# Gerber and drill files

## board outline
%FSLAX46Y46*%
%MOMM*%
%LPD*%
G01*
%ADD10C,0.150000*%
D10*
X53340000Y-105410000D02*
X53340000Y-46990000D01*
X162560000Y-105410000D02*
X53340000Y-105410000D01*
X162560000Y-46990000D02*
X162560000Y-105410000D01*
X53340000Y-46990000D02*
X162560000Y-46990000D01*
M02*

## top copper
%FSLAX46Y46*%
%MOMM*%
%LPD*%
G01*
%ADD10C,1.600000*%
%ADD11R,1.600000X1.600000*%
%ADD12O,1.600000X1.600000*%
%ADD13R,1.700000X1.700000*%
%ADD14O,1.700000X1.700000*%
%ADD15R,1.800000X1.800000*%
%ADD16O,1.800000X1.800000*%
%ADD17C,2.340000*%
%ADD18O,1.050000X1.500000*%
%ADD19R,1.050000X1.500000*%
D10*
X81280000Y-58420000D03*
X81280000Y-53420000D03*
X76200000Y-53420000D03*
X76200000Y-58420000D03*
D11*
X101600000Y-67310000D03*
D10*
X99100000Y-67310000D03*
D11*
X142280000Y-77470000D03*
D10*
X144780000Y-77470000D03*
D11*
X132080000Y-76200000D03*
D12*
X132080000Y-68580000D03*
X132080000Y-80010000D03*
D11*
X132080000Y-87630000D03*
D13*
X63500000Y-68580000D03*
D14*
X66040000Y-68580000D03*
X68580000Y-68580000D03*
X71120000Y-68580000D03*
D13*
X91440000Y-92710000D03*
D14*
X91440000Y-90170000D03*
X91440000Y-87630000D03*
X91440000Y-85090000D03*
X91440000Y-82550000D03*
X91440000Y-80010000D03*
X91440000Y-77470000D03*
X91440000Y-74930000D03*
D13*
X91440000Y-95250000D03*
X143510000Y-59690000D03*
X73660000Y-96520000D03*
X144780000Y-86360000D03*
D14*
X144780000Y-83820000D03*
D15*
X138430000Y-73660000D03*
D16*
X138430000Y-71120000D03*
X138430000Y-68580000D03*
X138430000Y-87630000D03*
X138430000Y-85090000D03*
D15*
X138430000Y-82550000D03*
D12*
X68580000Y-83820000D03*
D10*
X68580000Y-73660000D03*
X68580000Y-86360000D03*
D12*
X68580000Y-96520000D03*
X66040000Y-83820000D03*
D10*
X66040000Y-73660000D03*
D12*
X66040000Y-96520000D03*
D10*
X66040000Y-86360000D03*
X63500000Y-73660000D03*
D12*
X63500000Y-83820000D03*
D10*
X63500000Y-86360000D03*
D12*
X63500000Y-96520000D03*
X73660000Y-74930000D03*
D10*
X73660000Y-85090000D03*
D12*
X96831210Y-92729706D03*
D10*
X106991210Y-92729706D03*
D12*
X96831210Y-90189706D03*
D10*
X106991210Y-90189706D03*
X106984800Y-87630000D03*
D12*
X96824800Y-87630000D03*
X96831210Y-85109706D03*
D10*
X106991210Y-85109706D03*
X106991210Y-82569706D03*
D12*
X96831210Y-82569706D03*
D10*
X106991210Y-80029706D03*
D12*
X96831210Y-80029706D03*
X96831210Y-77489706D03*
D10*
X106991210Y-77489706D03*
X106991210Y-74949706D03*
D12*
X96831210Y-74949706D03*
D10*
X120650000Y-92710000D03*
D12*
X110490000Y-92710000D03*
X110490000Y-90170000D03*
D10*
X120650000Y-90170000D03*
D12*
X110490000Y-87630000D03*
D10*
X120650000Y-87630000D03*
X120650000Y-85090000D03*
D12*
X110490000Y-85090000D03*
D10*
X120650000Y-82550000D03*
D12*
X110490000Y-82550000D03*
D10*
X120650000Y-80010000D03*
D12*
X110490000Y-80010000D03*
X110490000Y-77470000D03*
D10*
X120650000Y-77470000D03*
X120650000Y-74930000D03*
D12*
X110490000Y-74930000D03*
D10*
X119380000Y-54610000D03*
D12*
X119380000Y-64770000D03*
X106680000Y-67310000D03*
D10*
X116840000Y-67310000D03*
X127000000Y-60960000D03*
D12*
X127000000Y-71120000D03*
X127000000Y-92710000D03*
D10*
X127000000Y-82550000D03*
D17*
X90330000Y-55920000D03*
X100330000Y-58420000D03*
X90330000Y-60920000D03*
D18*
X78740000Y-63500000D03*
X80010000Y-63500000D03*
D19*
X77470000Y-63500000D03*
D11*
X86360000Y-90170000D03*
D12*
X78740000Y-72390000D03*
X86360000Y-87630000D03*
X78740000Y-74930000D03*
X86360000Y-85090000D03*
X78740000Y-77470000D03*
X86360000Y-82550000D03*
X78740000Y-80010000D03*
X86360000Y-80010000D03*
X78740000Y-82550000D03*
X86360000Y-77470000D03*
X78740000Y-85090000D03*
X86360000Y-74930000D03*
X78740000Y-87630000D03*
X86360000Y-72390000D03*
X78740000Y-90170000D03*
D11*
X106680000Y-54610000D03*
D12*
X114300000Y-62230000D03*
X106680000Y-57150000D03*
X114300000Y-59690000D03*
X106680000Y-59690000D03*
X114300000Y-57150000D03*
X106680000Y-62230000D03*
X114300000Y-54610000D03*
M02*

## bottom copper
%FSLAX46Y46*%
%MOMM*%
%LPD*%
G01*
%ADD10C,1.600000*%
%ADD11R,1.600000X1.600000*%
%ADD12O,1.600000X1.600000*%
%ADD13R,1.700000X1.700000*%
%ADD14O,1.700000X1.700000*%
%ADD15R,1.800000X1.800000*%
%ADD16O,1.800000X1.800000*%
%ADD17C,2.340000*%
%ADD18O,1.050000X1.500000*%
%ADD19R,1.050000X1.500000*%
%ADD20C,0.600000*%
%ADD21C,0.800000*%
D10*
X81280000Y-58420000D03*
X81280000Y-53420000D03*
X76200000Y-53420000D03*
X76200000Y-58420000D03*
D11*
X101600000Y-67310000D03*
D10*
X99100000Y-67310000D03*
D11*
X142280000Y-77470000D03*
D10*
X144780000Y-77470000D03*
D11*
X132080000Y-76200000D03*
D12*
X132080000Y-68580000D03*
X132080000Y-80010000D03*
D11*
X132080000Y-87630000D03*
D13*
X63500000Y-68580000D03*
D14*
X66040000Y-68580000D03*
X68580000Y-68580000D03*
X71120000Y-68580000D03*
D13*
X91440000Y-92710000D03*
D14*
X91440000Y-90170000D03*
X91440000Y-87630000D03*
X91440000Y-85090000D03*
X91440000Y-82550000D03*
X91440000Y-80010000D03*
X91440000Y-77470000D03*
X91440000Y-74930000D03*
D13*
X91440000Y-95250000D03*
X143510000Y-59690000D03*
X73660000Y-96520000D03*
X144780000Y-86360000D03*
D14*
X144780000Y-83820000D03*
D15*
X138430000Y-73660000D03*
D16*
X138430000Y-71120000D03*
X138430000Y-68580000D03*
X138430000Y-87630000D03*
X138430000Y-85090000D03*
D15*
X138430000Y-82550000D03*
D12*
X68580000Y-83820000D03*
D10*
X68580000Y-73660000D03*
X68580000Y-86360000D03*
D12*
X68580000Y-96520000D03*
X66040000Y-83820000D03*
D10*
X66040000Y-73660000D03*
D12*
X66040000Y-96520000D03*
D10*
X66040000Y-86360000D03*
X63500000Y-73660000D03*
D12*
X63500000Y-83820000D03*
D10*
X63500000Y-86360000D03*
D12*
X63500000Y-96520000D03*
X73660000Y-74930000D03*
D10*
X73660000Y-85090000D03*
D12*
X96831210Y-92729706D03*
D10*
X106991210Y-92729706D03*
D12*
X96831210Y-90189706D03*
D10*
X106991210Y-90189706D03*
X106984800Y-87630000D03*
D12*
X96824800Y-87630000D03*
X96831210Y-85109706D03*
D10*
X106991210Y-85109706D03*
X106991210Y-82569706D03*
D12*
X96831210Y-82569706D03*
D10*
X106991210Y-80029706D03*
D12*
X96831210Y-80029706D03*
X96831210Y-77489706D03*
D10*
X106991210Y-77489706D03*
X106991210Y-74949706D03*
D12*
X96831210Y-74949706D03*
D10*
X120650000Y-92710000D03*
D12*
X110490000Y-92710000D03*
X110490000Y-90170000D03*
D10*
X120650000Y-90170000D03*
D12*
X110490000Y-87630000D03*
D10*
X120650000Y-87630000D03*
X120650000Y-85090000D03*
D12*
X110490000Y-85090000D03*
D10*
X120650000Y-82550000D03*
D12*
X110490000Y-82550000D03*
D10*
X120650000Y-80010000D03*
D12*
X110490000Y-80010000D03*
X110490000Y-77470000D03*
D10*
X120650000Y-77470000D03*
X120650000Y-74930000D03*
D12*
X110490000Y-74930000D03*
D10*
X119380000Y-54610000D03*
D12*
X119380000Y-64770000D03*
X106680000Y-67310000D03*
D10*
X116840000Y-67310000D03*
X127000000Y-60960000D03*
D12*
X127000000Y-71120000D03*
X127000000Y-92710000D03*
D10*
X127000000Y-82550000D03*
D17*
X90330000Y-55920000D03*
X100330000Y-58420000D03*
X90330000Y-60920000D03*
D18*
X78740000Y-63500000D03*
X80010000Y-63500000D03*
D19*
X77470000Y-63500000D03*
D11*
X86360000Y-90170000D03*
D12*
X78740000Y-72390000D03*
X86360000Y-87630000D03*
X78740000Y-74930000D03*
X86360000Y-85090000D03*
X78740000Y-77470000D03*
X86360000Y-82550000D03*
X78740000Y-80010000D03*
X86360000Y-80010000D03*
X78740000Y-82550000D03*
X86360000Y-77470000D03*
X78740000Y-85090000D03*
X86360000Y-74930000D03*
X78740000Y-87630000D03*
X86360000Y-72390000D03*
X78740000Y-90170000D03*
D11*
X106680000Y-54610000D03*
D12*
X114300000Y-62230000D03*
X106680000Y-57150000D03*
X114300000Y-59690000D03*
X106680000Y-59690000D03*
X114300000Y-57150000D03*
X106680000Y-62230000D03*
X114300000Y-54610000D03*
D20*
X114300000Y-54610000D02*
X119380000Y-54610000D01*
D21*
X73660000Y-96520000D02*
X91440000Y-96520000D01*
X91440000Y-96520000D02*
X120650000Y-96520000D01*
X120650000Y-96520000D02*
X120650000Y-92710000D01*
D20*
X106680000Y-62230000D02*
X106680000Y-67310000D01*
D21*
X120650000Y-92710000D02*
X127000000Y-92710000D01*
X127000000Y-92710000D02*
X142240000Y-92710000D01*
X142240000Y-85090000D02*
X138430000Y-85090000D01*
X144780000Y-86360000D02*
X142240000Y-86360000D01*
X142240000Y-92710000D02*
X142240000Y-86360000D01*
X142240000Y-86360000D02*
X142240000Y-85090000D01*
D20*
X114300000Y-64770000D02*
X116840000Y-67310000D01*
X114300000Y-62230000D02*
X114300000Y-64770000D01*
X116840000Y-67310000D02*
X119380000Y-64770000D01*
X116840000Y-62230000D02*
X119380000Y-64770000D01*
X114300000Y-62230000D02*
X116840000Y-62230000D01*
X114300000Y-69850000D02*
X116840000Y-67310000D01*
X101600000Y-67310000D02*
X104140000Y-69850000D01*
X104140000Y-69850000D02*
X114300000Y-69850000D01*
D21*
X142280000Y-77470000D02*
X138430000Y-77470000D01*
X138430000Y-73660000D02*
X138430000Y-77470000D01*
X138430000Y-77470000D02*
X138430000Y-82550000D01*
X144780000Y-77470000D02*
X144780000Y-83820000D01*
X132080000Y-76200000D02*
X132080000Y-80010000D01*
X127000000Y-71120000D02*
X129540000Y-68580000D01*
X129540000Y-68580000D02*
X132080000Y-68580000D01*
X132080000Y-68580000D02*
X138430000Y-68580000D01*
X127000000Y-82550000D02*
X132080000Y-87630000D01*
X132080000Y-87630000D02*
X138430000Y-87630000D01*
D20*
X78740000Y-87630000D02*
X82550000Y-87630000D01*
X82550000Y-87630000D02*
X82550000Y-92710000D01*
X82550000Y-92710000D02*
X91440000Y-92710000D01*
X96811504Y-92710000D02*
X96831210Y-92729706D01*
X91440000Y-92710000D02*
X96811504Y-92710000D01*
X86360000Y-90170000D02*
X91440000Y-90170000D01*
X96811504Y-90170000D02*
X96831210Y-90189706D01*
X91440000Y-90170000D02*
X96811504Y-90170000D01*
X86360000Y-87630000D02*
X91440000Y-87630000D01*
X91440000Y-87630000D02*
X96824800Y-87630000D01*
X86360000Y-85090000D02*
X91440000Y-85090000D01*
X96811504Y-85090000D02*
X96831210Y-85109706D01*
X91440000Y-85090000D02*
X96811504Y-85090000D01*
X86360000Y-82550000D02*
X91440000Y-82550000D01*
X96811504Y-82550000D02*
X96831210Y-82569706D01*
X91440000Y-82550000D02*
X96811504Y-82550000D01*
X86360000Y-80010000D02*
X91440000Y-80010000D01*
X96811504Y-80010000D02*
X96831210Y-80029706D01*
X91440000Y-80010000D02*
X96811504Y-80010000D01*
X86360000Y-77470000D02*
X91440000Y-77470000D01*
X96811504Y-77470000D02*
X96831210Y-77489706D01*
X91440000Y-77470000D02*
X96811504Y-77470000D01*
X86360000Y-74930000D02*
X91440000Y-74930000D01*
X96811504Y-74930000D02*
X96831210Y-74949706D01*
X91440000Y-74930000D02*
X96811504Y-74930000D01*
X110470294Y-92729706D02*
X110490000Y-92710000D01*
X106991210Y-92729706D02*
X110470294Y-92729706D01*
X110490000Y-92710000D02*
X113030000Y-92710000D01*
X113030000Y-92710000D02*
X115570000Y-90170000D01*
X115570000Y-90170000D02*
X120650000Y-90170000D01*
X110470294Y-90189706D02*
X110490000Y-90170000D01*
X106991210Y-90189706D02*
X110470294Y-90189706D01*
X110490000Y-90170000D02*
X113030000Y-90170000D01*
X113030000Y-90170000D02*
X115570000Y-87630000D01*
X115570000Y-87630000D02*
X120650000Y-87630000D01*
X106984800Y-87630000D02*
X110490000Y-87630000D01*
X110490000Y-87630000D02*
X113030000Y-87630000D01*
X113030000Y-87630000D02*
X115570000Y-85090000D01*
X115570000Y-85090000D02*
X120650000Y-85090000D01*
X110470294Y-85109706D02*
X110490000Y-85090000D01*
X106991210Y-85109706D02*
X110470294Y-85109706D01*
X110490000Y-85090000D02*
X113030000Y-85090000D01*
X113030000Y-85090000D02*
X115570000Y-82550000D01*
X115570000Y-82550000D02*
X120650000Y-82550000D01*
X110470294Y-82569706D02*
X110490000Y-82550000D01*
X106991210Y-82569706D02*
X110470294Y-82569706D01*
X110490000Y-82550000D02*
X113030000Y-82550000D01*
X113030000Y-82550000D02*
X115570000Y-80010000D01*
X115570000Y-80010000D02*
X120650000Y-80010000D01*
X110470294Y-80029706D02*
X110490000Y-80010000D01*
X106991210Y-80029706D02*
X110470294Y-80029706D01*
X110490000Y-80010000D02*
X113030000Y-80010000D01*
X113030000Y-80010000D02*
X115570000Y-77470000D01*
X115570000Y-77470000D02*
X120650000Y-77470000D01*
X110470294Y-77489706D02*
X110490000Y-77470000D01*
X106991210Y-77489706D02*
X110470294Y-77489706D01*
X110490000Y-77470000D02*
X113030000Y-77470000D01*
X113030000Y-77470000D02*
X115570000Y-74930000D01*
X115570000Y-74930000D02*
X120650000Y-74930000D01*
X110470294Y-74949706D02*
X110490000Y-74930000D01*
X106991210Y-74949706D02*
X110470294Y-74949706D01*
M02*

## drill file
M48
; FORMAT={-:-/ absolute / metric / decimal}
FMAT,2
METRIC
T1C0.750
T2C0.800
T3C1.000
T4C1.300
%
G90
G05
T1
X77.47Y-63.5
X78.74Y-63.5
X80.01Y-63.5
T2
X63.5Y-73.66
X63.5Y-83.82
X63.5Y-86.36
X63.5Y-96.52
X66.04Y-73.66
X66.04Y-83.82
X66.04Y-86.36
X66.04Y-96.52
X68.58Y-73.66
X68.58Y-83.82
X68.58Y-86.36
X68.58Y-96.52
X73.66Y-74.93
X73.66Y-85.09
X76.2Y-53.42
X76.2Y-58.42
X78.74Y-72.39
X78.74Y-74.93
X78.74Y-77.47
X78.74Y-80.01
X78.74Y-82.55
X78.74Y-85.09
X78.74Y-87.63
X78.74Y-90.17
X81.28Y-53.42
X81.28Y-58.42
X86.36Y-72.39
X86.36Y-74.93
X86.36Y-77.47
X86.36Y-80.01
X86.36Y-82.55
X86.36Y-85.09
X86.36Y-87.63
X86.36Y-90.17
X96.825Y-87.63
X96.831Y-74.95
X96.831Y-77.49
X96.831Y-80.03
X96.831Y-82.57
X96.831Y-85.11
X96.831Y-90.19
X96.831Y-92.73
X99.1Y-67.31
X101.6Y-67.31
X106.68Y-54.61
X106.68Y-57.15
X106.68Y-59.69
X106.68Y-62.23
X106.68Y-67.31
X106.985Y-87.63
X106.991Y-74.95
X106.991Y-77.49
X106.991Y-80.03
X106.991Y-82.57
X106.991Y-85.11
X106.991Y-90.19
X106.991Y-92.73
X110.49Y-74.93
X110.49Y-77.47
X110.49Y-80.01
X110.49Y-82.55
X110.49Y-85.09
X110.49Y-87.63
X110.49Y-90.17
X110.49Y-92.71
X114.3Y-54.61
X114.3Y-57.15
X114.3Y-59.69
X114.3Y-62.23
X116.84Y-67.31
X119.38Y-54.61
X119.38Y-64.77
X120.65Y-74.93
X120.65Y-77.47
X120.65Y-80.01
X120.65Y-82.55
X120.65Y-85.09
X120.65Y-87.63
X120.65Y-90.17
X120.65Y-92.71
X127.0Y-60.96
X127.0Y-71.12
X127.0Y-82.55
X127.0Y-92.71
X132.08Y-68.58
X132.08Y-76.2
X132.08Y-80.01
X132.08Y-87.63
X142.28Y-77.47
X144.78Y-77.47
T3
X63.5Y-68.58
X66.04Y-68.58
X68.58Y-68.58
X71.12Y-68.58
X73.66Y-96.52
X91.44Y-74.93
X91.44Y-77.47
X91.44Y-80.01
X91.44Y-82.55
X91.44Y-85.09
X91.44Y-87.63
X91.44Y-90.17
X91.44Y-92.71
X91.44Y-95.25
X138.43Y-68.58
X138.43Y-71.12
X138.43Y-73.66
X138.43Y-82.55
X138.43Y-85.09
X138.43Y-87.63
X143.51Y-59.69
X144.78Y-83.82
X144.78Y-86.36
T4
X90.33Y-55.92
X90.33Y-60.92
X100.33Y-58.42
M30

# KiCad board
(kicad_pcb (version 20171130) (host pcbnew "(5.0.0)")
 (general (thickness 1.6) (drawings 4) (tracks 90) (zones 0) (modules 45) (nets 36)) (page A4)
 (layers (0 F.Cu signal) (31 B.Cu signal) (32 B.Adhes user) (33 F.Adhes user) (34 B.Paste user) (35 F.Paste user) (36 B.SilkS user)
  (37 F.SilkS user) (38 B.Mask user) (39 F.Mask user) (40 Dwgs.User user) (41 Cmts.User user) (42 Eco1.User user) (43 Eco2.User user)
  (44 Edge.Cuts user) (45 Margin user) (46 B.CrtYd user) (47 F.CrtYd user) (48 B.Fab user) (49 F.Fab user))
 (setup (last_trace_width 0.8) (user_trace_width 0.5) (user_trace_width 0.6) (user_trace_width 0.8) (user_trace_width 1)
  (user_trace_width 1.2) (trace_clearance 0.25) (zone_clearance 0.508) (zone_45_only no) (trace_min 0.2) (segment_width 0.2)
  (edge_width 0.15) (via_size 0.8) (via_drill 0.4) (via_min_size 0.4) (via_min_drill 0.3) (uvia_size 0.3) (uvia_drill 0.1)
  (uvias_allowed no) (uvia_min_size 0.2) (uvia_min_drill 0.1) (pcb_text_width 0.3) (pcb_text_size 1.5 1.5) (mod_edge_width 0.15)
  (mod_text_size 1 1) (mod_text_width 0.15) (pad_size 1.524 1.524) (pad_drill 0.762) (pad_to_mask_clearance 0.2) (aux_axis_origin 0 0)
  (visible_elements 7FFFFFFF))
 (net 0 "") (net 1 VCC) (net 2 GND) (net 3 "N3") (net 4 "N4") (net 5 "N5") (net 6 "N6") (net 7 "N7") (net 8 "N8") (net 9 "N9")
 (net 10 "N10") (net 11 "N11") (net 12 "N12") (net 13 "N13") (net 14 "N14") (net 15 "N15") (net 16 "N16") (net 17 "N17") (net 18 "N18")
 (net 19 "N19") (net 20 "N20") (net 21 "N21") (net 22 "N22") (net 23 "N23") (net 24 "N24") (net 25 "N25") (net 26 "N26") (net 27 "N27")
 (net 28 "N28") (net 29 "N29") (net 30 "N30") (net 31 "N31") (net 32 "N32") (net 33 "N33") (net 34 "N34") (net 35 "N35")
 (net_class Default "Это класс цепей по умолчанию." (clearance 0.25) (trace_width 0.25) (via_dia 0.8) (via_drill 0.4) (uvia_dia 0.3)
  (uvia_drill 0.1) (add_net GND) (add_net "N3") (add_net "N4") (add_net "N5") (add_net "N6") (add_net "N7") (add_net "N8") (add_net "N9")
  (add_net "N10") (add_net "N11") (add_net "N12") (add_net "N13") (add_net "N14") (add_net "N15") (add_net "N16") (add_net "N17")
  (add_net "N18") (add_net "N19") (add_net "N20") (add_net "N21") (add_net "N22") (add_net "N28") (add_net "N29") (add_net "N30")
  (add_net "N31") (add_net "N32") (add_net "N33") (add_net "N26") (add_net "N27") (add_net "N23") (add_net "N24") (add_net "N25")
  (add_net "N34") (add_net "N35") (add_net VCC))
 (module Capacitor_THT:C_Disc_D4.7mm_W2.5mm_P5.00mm (layer F.Cu) (at 81.28 58.42 90)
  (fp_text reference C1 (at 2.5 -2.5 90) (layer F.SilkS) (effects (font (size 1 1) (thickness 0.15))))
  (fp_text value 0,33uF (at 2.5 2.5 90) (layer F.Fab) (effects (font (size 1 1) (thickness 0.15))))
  (pad 1 thru_hole circle (at 0 0 90) (size 1.6 1.6) (drill 0.8) (layers *.Cu *.Mask) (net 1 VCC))
  (pad 2 thru_hole circle (at 5 0 90) (size 1.6 1.6) (drill 0.8) (layers *.Cu *.Mask) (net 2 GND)))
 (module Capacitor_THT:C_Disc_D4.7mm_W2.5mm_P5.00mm (layer F.Cu) (at 76.2 58.42 90)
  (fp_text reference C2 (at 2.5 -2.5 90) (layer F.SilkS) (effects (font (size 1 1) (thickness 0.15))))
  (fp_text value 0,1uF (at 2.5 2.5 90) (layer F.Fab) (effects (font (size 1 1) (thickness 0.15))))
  (pad 2 thru_hole circle (at 5 0 90) (size 1.6 1.6) (drill 0.8) (layers *.Cu *.Mask) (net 2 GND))
  (pad 1 thru_hole circle (at 0 0 90) (size 1.6 1.6) (drill 0.8) (layers *.Cu *.Mask) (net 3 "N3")))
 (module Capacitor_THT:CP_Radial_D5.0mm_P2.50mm (layer F.Cu) (at 101.6 67.31 180)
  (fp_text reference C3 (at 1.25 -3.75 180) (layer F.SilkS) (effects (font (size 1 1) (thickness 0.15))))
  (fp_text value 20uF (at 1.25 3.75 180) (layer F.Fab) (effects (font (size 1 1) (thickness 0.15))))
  (pad 1 thru_hole rect (at 0 0 180) (size 1.6 1.6) (drill 0.8) (layers *.Cu *.Mask) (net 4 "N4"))
  (pad 2 thru_hole circle (at 2.5 0 180) (size 1.6 1.6) (drill 0.8) (layers *.Cu *.Mask) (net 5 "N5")))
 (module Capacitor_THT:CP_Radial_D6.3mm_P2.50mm (layer F.Cu) (at 142.28 77.47)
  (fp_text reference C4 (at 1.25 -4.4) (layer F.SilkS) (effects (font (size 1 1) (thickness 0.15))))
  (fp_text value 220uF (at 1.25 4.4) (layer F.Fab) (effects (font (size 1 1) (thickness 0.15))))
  (pad 1 thru_hole rect (at 0 0) (size 1.6 1.6) (drill 0.8) (layers *.Cu *.Mask) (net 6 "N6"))
  (pad 2 thru_hole circle (at 2.5 0) (size 1.6 1.6) (drill 0.8) (layers *.Cu *.Mask) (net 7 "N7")))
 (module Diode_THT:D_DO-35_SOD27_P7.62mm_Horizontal (layer F.Cu) (at 132.08 76.2 90)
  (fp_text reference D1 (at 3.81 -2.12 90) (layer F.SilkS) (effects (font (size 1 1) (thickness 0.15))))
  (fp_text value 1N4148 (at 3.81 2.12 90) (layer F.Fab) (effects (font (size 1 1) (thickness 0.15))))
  (pad 1 thru_hole rect (at 0 0 90) (size 1.6 1.6) (drill 0.8) (layers *.Cu *.Mask) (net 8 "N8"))
  (pad 2 thru_hole oval (at 7.62 0 90) (size 1.6 1.6) (drill 0.8) (layers *.Cu *.Mask) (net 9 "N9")))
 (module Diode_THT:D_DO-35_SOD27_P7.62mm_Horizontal (layer F.Cu) (at 132.08 87.63 90)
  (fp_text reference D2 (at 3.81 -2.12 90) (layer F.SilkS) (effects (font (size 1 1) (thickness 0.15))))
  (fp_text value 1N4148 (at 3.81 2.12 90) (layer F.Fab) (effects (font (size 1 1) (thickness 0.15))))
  (pad 2 thru_hole oval (at 7.62 0 90) (size 1.6 1.6) (drill 0.8) (layers *.Cu *.Mask) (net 8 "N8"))
  (pad 1 thru_hole rect (at 0 0 90) (size 1.6 1.6) (drill 0.8) (layers *.Cu *.Mask) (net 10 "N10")))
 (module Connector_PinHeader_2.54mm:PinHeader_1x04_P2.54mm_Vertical (layer F.Cu) (at 63.5 68.58 90)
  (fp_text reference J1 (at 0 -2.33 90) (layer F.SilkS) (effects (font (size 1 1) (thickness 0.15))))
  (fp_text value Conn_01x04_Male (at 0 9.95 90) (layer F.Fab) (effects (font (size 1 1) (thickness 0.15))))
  (pad 1 thru_hole rect (at 0 0 90) (size 1.7 1.7) (drill 1) (layers *.Cu *.Mask) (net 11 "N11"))
  (pad 2 thru_hole oval (at 0 2.54 90) (size 1.7 1.7) (drill 1) (layers *.Cu *.Mask) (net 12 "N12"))
  (pad 3 thru_hole oval (at 0 5.08 90) (size 1.7 1.7) (drill 1) (layers *.Cu *.Mask) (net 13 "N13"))
  (pad 4 thru_hole oval (at 0 7.62 90) (size 1.7 1.7) (drill 1) (layers *.Cu *.Mask) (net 2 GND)))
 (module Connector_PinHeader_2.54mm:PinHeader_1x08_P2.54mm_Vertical (layer F.Cu) (at 91.44 92.71 180)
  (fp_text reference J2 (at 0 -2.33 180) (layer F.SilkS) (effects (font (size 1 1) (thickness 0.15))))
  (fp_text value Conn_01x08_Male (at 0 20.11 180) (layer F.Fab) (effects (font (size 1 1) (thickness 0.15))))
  (pad 1 thru_hole rect (at 0 0 180) (size 1.7 1.7) (drill 1) (layers *.Cu *.Mask) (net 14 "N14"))
  (pad 2 thru_hole oval (at 0 2.54 180) (size 1.7 1.7) (drill 1) (layers *.Cu *.Mask) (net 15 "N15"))
  (pad 3 thru_hole oval (at 0 5.08 180) (size 1.7 1.7) (drill 1) (layers *.Cu *.Mask) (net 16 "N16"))
  (pad 4 thru_hole oval (at 0 7.62 180) (size 1.7 1.7) (drill 1) (layers *.Cu *.Mask) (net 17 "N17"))
  (pad 5 thru_hole oval (at 0 10.16 180) (size 1.7 1.7) (drill 1) (layers *.Cu *.Mask) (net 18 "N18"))
  (pad 6 thru_hole oval (at 0 12.7 180) (size 1.7 1.7) (drill 1) (layers *.Cu *.Mask) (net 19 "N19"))
  (pad 7 thru_hole oval (at 0 15.24 180) (size 1.7 1.7) (drill 1) (layers *.Cu *.Mask) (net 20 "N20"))
  (pad 8 thru_hole oval (at 0 17.78 180) (size 1.7 1.7) (drill 1) (layers *.Cu *.Mask) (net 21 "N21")))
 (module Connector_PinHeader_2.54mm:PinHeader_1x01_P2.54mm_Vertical (layer F.Cu) (at 91.44 95.25)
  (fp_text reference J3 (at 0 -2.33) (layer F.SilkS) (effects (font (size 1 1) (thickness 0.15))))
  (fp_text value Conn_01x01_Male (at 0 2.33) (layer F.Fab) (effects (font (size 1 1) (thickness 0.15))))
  (pad 1 thru_hole rect (at 0 0) (size 1.7 1.7) (drill 1) (layers *.Cu *.Mask) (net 2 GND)))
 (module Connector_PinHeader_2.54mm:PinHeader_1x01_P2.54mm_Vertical (layer F.Cu) (at 143.51 59.69)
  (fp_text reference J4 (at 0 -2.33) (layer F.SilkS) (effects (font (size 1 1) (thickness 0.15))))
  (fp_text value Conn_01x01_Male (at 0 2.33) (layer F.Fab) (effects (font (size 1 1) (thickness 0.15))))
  (pad 1 thru_hole rect (at 0 0) (size 1.7 1.7) (drill 1) (layers *.Cu *.Mask) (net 1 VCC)))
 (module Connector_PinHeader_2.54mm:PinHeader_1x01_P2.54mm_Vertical (layer F.Cu) (at 73.66 96.52)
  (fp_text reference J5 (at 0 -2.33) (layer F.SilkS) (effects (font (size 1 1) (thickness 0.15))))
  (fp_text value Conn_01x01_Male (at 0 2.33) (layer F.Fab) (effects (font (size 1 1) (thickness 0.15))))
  (pad 1 thru_hole rect (at 0 0) (size 1.7 1.7) (drill 1) (layers *.Cu *.Mask) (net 2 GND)))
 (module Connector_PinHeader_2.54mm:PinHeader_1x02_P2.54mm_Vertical (layer F.Cu) (at 144.78 86.36 180)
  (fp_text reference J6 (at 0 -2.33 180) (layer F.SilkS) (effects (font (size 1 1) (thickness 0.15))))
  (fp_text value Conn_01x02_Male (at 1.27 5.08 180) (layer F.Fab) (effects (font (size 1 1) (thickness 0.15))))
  (pad 1 thru_hole rect (at 0 0 180) (size 1.7 1.7) (drill 1) (layers *.Cu *.Mask) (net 2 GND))
  (pad 2 thru_hole oval (at 0 2.54 180) (size 1.7 1.7) (drill 1) (layers *.Cu *.Mask) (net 7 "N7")))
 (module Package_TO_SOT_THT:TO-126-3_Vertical (layer F.Cu) (at 138.43 73.66 90)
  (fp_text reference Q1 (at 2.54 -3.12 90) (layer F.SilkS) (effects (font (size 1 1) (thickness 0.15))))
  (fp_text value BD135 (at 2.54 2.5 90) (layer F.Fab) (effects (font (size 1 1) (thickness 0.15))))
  (pad 1 thru_hole rect (at 0 0 90) (size 1.8 1.8) (drill 1) (layers *.Cu *.Mask) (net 6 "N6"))
  (pad 2 thru_hole oval (at 2.54 0 90) (size 1.8 1.8) (drill 1) (layers *.Cu *.Mask) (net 1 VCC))
  (pad 3 thru_hole oval (at 5.08 0 90) (size 1.8 1.8) (drill 1) (layers *.Cu *.Mask) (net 9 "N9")))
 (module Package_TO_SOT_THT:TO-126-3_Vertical (layer F.Cu) (at 138.43 82.55 270)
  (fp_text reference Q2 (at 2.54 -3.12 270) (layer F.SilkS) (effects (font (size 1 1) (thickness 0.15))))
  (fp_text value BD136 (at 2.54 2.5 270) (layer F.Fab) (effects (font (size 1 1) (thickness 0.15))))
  (pad 3 thru_hole oval (at 5.08 0 270) (size 1.8 1.8) (drill 1) (layers *.Cu *.Mask) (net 10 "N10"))
  (pad 2 thru_hole oval (at 2.54 0 270) (size 1.8 1.8) (drill 1) (layers *.Cu *.Mask) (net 2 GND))
  (pad 1 thru_hole rect (at 0 0 270) (size 1.8 1.8) (drill 1) (layers *.Cu *.Mask) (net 6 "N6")))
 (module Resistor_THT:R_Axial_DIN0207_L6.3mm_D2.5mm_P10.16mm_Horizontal (layer F.Cu) (at 68.58 73.66 270)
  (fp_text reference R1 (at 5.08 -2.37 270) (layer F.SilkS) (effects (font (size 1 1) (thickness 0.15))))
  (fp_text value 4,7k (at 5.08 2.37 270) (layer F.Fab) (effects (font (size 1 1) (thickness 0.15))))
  (pad 2 thru_hole oval (at 10.16 0 270) (size 1.6 1.6) (drill 0.8) (layers *.Cu *.Mask) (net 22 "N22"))
  (pad 1 thru_hole circle (at 0 0 270) (size 1.6 1.6) (drill 0.8) (layers *.Cu *.Mask) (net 13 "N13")))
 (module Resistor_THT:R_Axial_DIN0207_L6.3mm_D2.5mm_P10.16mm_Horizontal (layer F.Cu) (at 68.58 86.36 270)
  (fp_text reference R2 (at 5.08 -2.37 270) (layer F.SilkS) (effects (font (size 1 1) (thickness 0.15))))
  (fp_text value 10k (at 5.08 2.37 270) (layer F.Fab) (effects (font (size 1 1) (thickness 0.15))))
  (pad 1 thru_hole circle (at 0 0 270) (size 1.6 1.6) (drill 0.8) (layers *.Cu *.Mask) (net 22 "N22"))
  (pad 2 thru_hole oval (at 10.16 0 270) (size 1.6 1.6) (drill 0.8) (layers *.Cu *.Mask) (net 2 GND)))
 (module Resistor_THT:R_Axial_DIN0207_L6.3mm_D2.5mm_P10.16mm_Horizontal (layer F.Cu) (at 66.04 73.66 270)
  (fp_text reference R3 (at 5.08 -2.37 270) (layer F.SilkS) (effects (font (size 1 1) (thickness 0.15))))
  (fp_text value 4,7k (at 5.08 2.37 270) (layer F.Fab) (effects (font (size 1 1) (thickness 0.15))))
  (pad 2 thru_hole oval (at 10.16 0 270) (size 1.6 1.6) (drill 0.8) (layers *.Cu *.Mask) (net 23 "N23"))
  (pad 1 thru_hole circle (at 0 0 270) (size 1.6 1.6) (drill 0.8) (layers *.Cu *.Mask) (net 12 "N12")))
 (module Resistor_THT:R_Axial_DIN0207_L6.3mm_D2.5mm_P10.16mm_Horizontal (layer F.Cu) (at 66.04 86.36 270)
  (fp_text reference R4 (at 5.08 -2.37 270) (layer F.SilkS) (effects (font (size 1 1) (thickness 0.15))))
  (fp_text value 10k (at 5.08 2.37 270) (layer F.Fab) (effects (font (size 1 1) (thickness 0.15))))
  (pad 2 thru_hole oval (at 10.16 0 270) (size 1.6 1.6) (drill 0.8) (layers *.Cu *.Mask) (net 2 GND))
  (pad 1 thru_hole circle (at 0 0 270) (size 1.6 1.6) (drill 0.8) (layers *.Cu *.Mask) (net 23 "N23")))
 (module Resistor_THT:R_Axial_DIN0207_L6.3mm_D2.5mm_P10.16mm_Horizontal (layer F.Cu) (at 63.5 73.66 270)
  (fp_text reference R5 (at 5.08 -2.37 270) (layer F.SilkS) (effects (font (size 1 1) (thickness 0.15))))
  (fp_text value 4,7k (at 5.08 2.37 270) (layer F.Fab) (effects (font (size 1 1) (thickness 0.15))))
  (pad 1 thru_hole circle (at 0 0 270) (size 1.6 1.6) (drill 0.8) (layers *.Cu *.Mask) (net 11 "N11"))
  (pad 2 thru_hole oval (at 10.16 0 270) (size 1.6 1.6) (drill 0.8) (layers *.Cu *.Mask) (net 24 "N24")))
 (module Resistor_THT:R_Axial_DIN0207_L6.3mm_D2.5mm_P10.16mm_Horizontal (layer F.Cu) (at 63.5 86.36 270)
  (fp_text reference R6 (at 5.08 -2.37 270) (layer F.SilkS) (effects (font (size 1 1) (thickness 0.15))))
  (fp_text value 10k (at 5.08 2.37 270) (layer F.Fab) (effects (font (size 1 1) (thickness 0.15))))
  (pad 1 thru_hole circle (at 0 0 270) (size 1.6 1.6) (drill 0.8) (layers *.Cu *.Mask) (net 24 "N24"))
  (pad 2 thru_hole oval (at 10.16 0 270) (size 1.6 1.6) (drill 0.8) (layers *.Cu *.Mask) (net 2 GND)))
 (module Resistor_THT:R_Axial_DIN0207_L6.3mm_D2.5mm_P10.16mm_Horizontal (layer F.Cu) (at 73.66 85.09 90)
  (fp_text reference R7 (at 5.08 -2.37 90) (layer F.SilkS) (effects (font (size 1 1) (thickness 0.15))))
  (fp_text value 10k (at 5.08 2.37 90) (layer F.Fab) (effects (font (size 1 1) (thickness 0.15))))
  (pad 2 thru_hole oval (at 10.16 0 90) (size 1.6 1.6) (drill 0.8) (layers *.Cu *.Mask) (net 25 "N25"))
  (pad 1 thru_hole circle (at 0 0 90) (size 1.6 1.6) (drill 0.8) (layers *.Cu *.Mask) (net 3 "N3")))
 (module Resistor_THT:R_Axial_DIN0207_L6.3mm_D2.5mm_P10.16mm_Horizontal (layer F.Cu) (at 106.99121 92.729706 180)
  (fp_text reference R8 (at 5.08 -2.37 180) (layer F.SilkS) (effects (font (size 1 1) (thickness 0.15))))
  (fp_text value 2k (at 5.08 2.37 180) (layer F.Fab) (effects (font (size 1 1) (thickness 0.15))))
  (pad 2 thru_hole oval (at 10.16 0 180) (size 1.6 1.6) (drill 0.8) (layers *.Cu *.Mask) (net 14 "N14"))
  (pad 1 thru_hole circle (at 0 0 180) (size 1.6 1.6) (drill 0.8) (layers *.Cu *.Mask) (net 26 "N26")))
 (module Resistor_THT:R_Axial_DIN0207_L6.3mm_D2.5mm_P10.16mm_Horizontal (layer F.Cu) (at 106.99121 90.189706 180)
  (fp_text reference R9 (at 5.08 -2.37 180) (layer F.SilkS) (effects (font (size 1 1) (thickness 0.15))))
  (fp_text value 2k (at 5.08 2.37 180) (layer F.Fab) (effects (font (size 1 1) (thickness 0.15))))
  (pad 2 thru_hole oval (at 10.16 0 180) (size 1.6 1.6) (drill 0.8) (layers *.Cu *.Mask) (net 15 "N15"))
  (pad 1 thru_hole circle (at 0 0 180) (size 1.6 1.6) (drill 0.8) (layers *.Cu *.Mask) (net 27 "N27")))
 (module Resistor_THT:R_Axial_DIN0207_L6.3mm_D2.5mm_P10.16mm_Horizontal (layer F.Cu) (at 106.9848 87.63 180)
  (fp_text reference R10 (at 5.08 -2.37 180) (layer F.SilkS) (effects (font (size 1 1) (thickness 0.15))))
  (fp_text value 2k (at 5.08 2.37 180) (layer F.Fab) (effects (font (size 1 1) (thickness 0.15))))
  (pad 1 thru_hole circle (at 0 0 180) (size 1.6 1.6) (drill 0.8) (layers *.Cu *.Mask) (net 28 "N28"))
  (pad 2 thru_hole oval (at 10.16 0 180) (size 1.6 1.6) (drill 0.8) (layers *.Cu *.Mask) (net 16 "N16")))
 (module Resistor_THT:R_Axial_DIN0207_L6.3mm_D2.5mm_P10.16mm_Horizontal (layer F.Cu) (at 106.99121 85.109706 180)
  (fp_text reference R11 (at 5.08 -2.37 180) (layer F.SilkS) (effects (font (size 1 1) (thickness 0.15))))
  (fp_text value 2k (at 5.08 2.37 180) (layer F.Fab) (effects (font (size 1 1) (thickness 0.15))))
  (pad 2 thru_hole oval (at 10.16 0 180) (size 1.6 1.6) (drill 0.8) (layers *.Cu *.Mask) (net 17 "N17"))
  (pad 1 thru_hole circle (at 0 0 180) (size 1.6 1.6) (drill 0.8) (layers *.Cu *.Mask) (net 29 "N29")))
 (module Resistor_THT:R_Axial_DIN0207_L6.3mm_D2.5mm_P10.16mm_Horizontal (layer F.Cu) (at 106.99121 82.569706 180)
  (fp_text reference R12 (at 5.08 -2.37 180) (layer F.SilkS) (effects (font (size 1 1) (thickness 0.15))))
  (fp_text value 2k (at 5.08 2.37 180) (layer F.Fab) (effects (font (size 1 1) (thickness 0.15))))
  (pad 1 thru_hole circle (at 0 0 180) (size 1.6 1.6) (drill 0.8) (layers *.Cu *.Mask) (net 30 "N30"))
  (pad 2 thru_hole oval (at 10.16 0 180) (size 1.6 1.6) (drill 0.8) (layers *.Cu *.Mask) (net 18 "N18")))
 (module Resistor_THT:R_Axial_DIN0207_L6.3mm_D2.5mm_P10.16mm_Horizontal (layer F.Cu) (at 106.99121 80.029706 180)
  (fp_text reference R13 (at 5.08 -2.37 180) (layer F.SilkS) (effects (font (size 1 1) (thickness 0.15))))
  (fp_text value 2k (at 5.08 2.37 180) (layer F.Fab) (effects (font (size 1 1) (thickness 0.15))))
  (pad 1 thru_hole circle (at 0 0 180) (size 1.6 1.6) (drill 0.8) (layers *.Cu *.Mask) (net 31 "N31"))
  (pad 2 thru_hole oval (at 10.16 0 180) (size 1.6 1.6) (drill 0.8) (layers *.Cu *.Mask) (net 19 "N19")))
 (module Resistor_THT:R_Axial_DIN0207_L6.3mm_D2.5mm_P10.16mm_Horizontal (layer F.Cu) (at 106.99121 77.489706 180)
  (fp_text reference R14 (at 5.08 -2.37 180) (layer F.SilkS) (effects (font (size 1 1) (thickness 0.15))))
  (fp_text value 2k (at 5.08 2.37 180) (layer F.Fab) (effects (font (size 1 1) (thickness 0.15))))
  (pad 2 thru_hole oval (at 10.16 0 180) (size 1.6 1.6) (drill 0.8) (layers *.Cu *.Mask) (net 20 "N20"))
  (pad 1 thru_hole circle (at 0 0 180) (size 1.6 1.6) (drill 0.8) (layers *.Cu *.Mask) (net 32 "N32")))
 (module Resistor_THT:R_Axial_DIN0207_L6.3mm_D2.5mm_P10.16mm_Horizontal (layer F.Cu) (at 106.99121 74.949706 180)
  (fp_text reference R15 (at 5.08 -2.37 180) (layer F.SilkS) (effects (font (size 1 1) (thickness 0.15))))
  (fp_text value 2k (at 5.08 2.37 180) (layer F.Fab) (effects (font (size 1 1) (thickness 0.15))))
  (pad 1 thru_hole circle (at 0 0 180) (size 1.6 1.6) (drill 0.8) (layers *.Cu *.Mask) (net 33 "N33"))
  (pad 2 thru_hole oval (at 10.16 0 180) (size 1.6 1.6) (drill 0.8) (layers *.Cu *.Mask) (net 21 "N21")))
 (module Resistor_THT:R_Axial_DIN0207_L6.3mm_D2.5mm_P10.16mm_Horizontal (layer F.Cu) (at 120.65 92.71 180)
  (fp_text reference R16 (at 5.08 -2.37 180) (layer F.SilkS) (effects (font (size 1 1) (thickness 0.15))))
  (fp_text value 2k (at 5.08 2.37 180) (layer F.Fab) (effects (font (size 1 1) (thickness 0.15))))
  (pad 1 thru_hole circle (at 0 0 180) (size 1.6 1.6) (drill 0.8) (layers *.Cu *.Mask) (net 2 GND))
  (pad 2 thru_hole oval (at 10.16 0 180) (size 1.6 1.6) (drill 0.8) (layers *.Cu *.Mask) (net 26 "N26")))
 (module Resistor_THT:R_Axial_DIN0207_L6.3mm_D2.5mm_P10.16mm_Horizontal (layer F.Cu) (at 120.65 90.17 180)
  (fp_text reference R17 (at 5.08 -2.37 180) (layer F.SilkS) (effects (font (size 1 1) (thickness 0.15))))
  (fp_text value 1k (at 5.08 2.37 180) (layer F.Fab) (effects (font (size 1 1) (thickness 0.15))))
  (pad 2 thru_hole oval (at 10.16 0 180) (size 1.6 1.6) (drill 0.8) (layers *.Cu *.Mask) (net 27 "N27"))
  (pad 1 thru_hole circle (at 0 0 180) (size 1.6 1.6) (drill 0.8) (layers *.Cu *.Mask) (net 26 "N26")))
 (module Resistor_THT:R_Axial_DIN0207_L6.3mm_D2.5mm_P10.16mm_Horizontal (layer F.Cu) (at 120.65 87.63 180)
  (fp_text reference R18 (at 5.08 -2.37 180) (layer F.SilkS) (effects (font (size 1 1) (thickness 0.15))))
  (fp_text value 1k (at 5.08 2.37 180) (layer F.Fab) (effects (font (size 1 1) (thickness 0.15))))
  (pad 2 thru_hole oval (at 10.16 0 180) (size 1.6 1.6) (drill 0.8) (layers *.Cu *.Mask) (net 28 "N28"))
  (pad 1 thru_hole circle (at 0 0 180) (size 1.6 1.6) (drill 0.8) (layers *.Cu *.Mask) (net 27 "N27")))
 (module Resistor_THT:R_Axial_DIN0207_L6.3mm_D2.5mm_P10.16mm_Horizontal (layer F.Cu) (at 120.65 85.09 180)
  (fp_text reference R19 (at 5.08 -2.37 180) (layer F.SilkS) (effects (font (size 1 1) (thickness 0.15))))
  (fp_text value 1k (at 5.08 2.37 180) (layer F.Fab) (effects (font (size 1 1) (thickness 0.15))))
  (pad 1 thru_hole circle (at 0 0 180) (size 1.6 1.6) (drill 0.8) (layers *.Cu *.Mask) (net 28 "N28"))
  (pad 2 thru_hole oval (at 10.16 0 180) (size 1.6 1.6) (drill 0.8) (layers *.Cu *.Mask) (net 29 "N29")))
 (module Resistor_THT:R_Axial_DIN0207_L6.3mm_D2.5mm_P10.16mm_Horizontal (layer F.Cu) (at 120.65 82.55 180)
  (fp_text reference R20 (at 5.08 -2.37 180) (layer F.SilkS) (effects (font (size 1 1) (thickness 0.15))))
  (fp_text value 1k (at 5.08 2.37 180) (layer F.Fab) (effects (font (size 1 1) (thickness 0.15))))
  (pad 1 thru_hole circle (at 0 0 180) (size 1.6 1.6) (drill 0.8) (layers *.Cu *.Mask) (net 29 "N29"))
  (pad 2 thru_hole oval (at 10.16 0 180) (size 1.6 1.6) (drill 0.8) (layers *.Cu *.Mask) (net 30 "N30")))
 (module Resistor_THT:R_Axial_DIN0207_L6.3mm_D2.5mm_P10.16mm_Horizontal (layer F.Cu) (at 120.65 80.01 180)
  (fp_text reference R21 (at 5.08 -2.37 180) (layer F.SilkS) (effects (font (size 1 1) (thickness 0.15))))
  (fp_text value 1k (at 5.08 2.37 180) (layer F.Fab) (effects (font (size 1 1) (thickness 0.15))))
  (pad 1 thru_hole circle (at 0 0 180) (size 1.6 1.6) (drill 0.8) (layers *.Cu *.Mask) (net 30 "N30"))
  (pad 2 thru_hole oval (at 10.16 0 180) (size 1.6 1.6) (drill 0.8) (layers *.Cu *.Mask) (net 31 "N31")))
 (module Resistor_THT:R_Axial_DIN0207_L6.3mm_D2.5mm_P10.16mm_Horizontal (layer F.Cu) (at 120.65 77.47 180)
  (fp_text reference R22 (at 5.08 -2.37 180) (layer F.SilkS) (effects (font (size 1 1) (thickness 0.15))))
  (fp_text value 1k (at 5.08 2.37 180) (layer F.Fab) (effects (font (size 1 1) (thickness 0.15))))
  (pad 2 thru_hole oval (at 10.16 0 180) (size 1.6 1.6) (drill 0.8) (layers *.Cu *.Mask) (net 32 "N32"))
  (pad 1 thru_hole circle (at 0 0 180) (size 1.6 1.6) (drill 0.8) (layers *.Cu *.Mask) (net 31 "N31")))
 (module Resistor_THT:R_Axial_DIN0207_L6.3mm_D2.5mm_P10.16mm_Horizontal (layer F.Cu) (at 120.65 74.93 180)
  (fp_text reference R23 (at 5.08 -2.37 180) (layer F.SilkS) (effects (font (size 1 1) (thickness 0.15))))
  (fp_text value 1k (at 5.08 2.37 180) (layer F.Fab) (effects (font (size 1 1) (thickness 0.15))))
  (pad 1 thru_hole circle (at 0 0 180) (size 1.6 1.6) (drill 0.8) (layers *.Cu *.Mask) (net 32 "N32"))
  (pad 2 thru_hole oval (at 10.16 0 180) (size 1.6 1.6) (drill 0.8) (layers *.Cu *.Mask) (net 33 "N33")))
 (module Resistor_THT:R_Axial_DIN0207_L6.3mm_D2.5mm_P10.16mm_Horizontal (layer F.Cu) (at 119.38 54.61 270)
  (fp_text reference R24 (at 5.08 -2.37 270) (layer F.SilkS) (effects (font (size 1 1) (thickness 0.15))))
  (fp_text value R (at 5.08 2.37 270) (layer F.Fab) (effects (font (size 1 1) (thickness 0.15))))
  (pad 1 thru_hole circle (at 0 0 270) (size 1.6 1.6) (drill 0.8) (layers *.Cu *.Mask) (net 1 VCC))
  (pad 2 thru_hole oval (at 10.16 0 270) (size 1.6 1.6) (drill 0.8) (layers *.Cu *.Mask) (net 4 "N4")))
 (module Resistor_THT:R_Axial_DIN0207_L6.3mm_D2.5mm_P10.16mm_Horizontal (layer F.Cu) (at 116.84 67.31 180)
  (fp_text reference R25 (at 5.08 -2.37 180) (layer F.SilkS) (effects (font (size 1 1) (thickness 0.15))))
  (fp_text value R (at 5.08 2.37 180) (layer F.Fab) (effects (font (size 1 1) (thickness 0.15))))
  (pad 2 thru_hole oval (at 10.16 0 180) (size 1.6 1.6) (drill 0.8) (layers *.Cu *.Mask) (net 2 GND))
  (pad 1 thru_hole circle (at 0 0 180) (size 1.6 1.6) (drill 0.8) (layers *.Cu *.Mask) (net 4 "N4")))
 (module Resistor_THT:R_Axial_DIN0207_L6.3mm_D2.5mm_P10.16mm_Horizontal (layer F.Cu) (at 127 60.96 270)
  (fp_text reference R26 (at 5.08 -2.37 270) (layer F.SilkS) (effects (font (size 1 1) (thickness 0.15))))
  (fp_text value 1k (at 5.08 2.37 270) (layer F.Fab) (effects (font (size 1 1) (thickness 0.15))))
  (pad 1 thru_hole circle (at 0 0 270) (size 1.6 1.6) (drill 0.8) (layers *.Cu *.Mask) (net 1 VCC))
  (pad 2 thru_hole oval (at 10.16 0 270) (size 1.6 1.6) (drill 0.8) (layers *.Cu *.Mask) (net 9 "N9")))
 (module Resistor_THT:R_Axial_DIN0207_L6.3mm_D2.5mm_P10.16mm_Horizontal (layer F.Cu) (at 127 82.55 270)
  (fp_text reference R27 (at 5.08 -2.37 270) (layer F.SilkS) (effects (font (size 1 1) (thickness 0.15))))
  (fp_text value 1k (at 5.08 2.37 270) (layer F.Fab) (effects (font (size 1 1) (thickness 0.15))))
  (pad 2 thru_hole oval (at 10.16 0 270) (size 1.6 1.6) (drill 0.8) (layers *.Cu *.Mask) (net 2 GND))
  (pad 1 thru_hole circle (at 0 0 270) (size 1.6 1.6) (drill 0.8) (layers *.Cu *.Mask) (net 10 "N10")))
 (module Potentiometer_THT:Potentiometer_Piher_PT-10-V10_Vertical (layer F.Cu) (at 90.33 60.92)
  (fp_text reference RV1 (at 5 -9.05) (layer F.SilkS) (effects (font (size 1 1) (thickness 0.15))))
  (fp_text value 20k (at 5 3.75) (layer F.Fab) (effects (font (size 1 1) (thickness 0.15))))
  (pad 3 thru_hole circle (at 0 -5) (size 2.34 2.34) (drill 1.3) (layers *.Cu *.Mask) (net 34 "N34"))
  (pad 2 thru_hole circle (at 10 -2.5) (size 2.34 2.34) (drill 1.3) (layers *.Cu *.Mask) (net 5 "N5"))
  (pad 1 thru_hole circle (at 0 0) (size 2.34 2.34) (drill 1.3) (layers *.Cu *.Mask) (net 2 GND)))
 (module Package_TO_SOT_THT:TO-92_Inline (layer F.Cu) (at 77.47 63.5)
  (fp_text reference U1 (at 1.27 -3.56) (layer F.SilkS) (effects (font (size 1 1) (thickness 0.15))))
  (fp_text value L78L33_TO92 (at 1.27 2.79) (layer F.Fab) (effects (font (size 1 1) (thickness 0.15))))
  (pad 2 thru_hole oval (at 1.27 0) (size 1.05 1.5) (drill 0.75) (layers *.Cu *.Mask) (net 2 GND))
  (pad 3 thru_hole oval (at 2.54 0) (size 1.05 1.5) (drill 0.75) (layers *.Cu *.Mask) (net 1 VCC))
  (pad 1 thru_hole rect (at 0 0) (size 1.05 1.5) (drill 0.75) (layers *.Cu *.Mask) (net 3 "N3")))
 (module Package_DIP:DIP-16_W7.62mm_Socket (layer F.Cu) (at 86.36 90.17 180)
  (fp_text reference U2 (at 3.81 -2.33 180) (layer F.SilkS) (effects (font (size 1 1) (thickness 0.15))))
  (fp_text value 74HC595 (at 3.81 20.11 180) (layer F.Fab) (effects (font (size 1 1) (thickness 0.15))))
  (pad 1 thru_hole rect (at 0 0 180) (size 1.6 1.6) (drill 0.8) (layers *.Cu *.Mask) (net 15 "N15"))
  (pad 9 thru_hole oval (at 7.62 17.78 180) (size 1.6 1.6) (drill 0.8) (layers *.Cu *.Mask) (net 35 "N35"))
  (pad 2 thru_hole oval (at 0 2.54 180) (size 1.6 1.6) (drill 0.8) (layers *.Cu *.Mask) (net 16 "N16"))
  (pad 10 thru_hole oval (at 7.62 15.24 180) (size 1.6 1.6) (drill 0.8) (layers *.Cu *.Mask) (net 25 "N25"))
  (pad 3 thru_hole oval (at 0 5.08 180) (size 1.6 1.6) (drill 0.8) (layers *.Cu *.Mask) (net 17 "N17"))
  (pad 11 thru_hole oval (at 7.62 12.7 180) (size 1.6 1.6) (drill 0.8) (layers *.Cu *.Mask) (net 23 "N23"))
  (pad 4 thru_hole oval (at 0 7.62 180) (size 1.6 1.6) (drill 0.8) (layers *.Cu *.Mask) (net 18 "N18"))
  (pad 12 thru_hole oval (at 7.62 10.16 180) (size 1.6 1.6) (drill 0.8) (layers *.Cu *.Mask) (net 24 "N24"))
  (pad 5 thru_hole oval (at 0 10.16 180) (size 1.6 1.6) (drill 0.8) (layers *.Cu *.Mask) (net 19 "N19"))
  (pad 13 thru_hole oval (at 7.62 7.62 180) (size 1.6 1.6) (drill 0.8) (layers *.Cu *.Mask) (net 2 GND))
  (pad 6 thru_hole oval (at 0 12.7 180) (size 1.6 1.6) (drill 0.8) (layers *.Cu *.Mask) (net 20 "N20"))
  (pad 14 thru_hole oval (at 7.62 5.08 180) (size 1.6 1.6) (drill 0.8) (layers *.Cu *.Mask) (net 22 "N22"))
  (pad 7 thru_hole oval (at 0 15.24 180) (size 1.6 1.6) (drill 0.8) (layers *.Cu *.Mask) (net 21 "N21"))
  (pad 15 thru_hole oval (at 7.62 2.54 180) (size 1.6 1.6) (drill 0.8) (layers *.Cu *.Mask) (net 14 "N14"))
  (pad 8 thru_hole oval (at 0 17.78 180) (size 1.6 1.6) (drill 0.8) (layers *.Cu *.Mask) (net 2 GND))
  (pad 16 thru_hole oval (at 7.62 0 180) (size 1.6 1.6) (drill 0.8) (layers *.Cu *.Mask) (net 3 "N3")))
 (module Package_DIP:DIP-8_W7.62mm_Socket (layer F.Cu) (at 106.68 54.61)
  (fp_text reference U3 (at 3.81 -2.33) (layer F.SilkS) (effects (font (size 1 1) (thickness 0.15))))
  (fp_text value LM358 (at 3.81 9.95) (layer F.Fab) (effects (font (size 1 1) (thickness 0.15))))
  (pad 1 thru_hole rect (at 0 0) (size 1.6 1.6) (drill 0.8) (layers *.Cu *.Mask) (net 34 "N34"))
  (pad 5 thru_hole oval (at 7.62 7.62) (size 1.6 1.6) (drill 0.8) (layers *.Cu *.Mask) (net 4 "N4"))
  (pad 2 thru_hole oval (at 0 2.54) (size 1.6 1.6) (drill 0.8) (layers *.Cu *.Mask) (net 34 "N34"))
  (pad 6 thru_hole oval (at 7.62 5.08) (size 1.6 1.6) (drill 0.8) (layers *.Cu *.Mask) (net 6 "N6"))
  (pad 3 thru_hole oval (at 0 5.08) (size 1.6 1.6) (drill 0.8) (layers *.Cu *.Mask) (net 33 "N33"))
  (pad 7 thru_hole oval (at 7.62 2.54) (size 1.6 1.6) (drill 0.8) (layers *.Cu *.Mask) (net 8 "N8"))
  (pad 4 thru_hole oval (at 0 7.62) (size 1.6 1.6) (drill 0.8) (layers *.Cu *.Mask) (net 2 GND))
  (pad 8 thru_hole oval (at 7.62 0) (size 1.6 1.6) (drill 0.8) (layers *.Cu *.Mask) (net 1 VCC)))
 (gr_line (start 53.34 105.41) (end 53.34 46.99) (layer Edge.Cuts) (width 0.15))
 (gr_line (start 162.56 105.41) (end 53.34 105.41) (layer Edge.Cuts) (width 0.15))
 (gr_line (start 162.56 46.99) (end 162.56 105.41) (layer Edge.Cuts) (width 0.15))
 (gr_line (start 53.34 46.99) (end 162.56 46.99) (layer Edge.Cuts) (width 0.15))
 (segment (start 114.3 54.61) (end 119.38 54.61) (width 0.6) (layer B.Cu) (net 1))
 (segment (start 73.66 96.52) (end 91.44 96.52) (width 0.8) (layer B.Cu) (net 2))
 (segment (start 91.44 96.52) (end 120.65 96.52) (width 0.8) (layer B.Cu) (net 2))
 (segment (start 120.65 96.52) (end 120.65 92.71) (width 0.8) (layer B.Cu) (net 2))
 (segment (start 106.68 62.23) (end 106.68 67.31) (width 0.6) (layer B.Cu) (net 2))
 (segment (start 120.65 92.71) (end 127 92.71) (width 0.8) (layer B.Cu) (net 2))
 (segment (start 127 92.71) (end 142.24 92.71) (width 0.8) (layer B.Cu) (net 2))
 (segment (start 142.24 85.09) (end 138.43 85.09) (width 0.8) (layer B.Cu) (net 2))
 (segment (start 144.78 86.36) (end 142.24 86.36) (width 0.8) (layer B.Cu) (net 2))
 (segment (start 142.24 92.71) (end 142.24 86.36) (width 0.8) (layer B.Cu) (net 2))
 (segment (start 142.24 86.36) (end 142.24 85.09) (width 0.8) (layer B.Cu) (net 2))
 (segment (start 114.3 64.77) (end 116.84 67.31) (width 0.6) (layer B.Cu) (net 4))
 (segment (start 114.3 62.23) (end 114.3 64.77) (width 0.6) (layer B.Cu) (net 4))
 (segment (start 116.84 67.31) (end 119.38 64.77) (width 0.6) (layer B.Cu) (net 4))
 (segment (start 116.84 62.23) (end 119.38 64.77) (width 0.6) (layer B.Cu) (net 4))
 (segment (start 114.3 62.23) (end 116.84 62.23) (width 0.6) (layer B.Cu) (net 4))
 (segment (start 114.3 69.85) (end 116.84 67.31) (width 0.6) (layer B.Cu) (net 4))
 (segment (start 101.6 67.31) (end 104.14 69.85) (width 0.6) (layer B.Cu) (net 4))
 (segment (start 104.14 69.85) (end 114.3 69.85) (width 0.6) (layer B.Cu) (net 4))
 (segment (start 142.28 77.47) (end 138.43 77.47) (width 0.8) (layer B.Cu) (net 6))
 (segment (start 138.43 73.66) (end 138.43 77.47) (width 0.8) (layer B.Cu) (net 6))
 (segment (start 138.43 77.47) (end 138.43 82.55) (width 0.8) (layer B.Cu) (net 6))
 (segment (start 144.78 77.47) (end 144.78 83.82) (width 0.8) (layer B.Cu) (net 7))
 (segment (start 132.08 76.2) (end 132.08 80.01) (width 0.8) (layer B.Cu) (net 8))
 (segment (start 127 71.12) (end 129.54 68.58) (width 0.8) (layer B.Cu) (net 9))
 (segment (start 129.54 68.58) (end 132.08 68.58) (width 0.8) (layer B.Cu) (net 9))
 (segment (start 132.08 68.58) (end 138.43 68.58) (width 0.8) (layer B.Cu) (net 9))
 (segment (start 127 82.55) (end 132.08 87.63) (width 0.8) (layer B.Cu) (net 10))
 (segment (start 132.08 87.63) (end 138.43 87.63) (width 0.8) (layer B.Cu) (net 10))
 (segment (start 78.74 87.63) (end 82.55 87.63) (width 0.6) (layer B.Cu) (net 14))
 (segment (start 82.55 87.63) (end 82.55 92.71) (width 0.6) (layer B.Cu) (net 14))
 (segment (start 82.55 92.71) (end 91.44 92.71) (width 0.6) (layer B.Cu) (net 14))
 (segment (start 96.811504 92.71) (end 96.83121 92.729706) (width 0.6) (layer B.Cu) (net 14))
 (segment (start 91.44 92.71) (end 96.811504 92.71) (width 0.6) (layer B.Cu) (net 14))
 (segment (start 86.36 90.17) (end 91.44 90.17) (width 0.6) (layer B.Cu) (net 15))
 (segment (start 96.811504 90.17) (end 96.83121 90.189706) (width 0.6) (layer B.Cu) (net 15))
 (segment (start 91.44 90.17) (end 96.811504 90.17) (width 0.6) (layer B.Cu) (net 15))
 (segment (start 86.36 87.63) (end 91.44 87.63) (width 0.6) (layer B.Cu) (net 16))
 (segment (start 91.44 87.63) (end 96.8248 87.63) (width 0.6) (layer B.Cu) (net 16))
 (segment (start 86.36 85.09) (end 91.44 85.09) (width 0.6) (layer B.Cu) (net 17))
 (segment (start 96.811504 85.09) (end 96.83121 85.109706) (width 0.6) (layer B.Cu) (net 17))
 (segment (start 91.44 85.09) (end 96.811504 85.09) (width 0.6) (layer B.Cu) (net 17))
 (segment (start 86.36 82.55) (end 91.44 82.55) (width 0.6) (layer B.Cu) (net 18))
 (segment (start 96.811504 82.55) (end 96.83121 82.569706) (width 0.6) (layer B.Cu) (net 18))
 (segment (start 91.44 82.55) (end 96.811504 82.55) (width 0.6) (layer B.Cu) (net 18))
 (segment (start 86.36 80.01) (end 91.44 80.01) (width 0.6) (layer B.Cu) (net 19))
 (segment (start 96.811504 80.01) (end 96.83121 80.029706) (width 0.6) (layer B.Cu) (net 19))
 (segment (start 91.44 80.01) (end 96.811504 80.01) (width 0.6) (layer B.Cu) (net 19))
 (segment (start 86.36 77.47) (end 91.44 77.47) (width 0.6) (layer B.Cu) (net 20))
 (segment (start 96.811504 77.47) (end 96.83121 77.489706) (width 0.6) (layer B.Cu) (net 20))
 (segment (start 91.44 77.47) (end 96.811504 77.47) (width 0.6) (layer B.Cu) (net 20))
 (segment (start 86.36 74.93) (end 91.44 74.93) (width 0.6) (layer B.Cu) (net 21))
 (segment (start 96.811504 74.93) (end 96.83121 74.949706) (width 0.6) (layer B.Cu) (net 21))
 (segment (start 91.44 74.93) (end 96.811504 74.93) (width 0.6) (layer B.Cu) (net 21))
 (segment (start 110.470294 92.729706) (end 110.49 92.71) (width 0.6) (layer B.Cu) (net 26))
 (segment (start 106.99121 92.729706) (end 110.470294 92.729706) (width 0.6) (layer B.Cu) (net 26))
 (segment (start 110.49 92.71) (end 113.03 92.71) (width 0.6) (layer B.Cu) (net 26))
 (segment (start 113.03 92.71) (end 115.57 90.17) (width 0.6) (layer B.Cu) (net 26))
 (segment (start 115.57 90.17) (end 120.65 90.17) (width 0.6) (layer B.Cu) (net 26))
 (segment (start 110.470294 90.189706) (end 110.49 90.17) (width 0.6) (layer B.Cu) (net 27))
 (segment (start 106.99121 90.189706) (end 110.470294 90.189706) (width 0.6) (layer B.Cu) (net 27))
 (segment (start 110.49 90.17) (end 113.03 90.17) (width 0.6) (layer B.Cu) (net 27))
 (segment (start 113.03 90.17) (end 115.57 87.63) (width 0.6) (layer B.Cu) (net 27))
 (segment (start 115.57 87.63) (end 120.65 87.63) (width 0.6) (layer B.Cu) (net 27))
 (segment (start 106.9848 87.63) (end 110.49 87.63) (width 0.6) (layer B.Cu) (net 28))
 (segment (start 110.49 87.63) (end 113.03 87.63) (width 0.6) (layer B.Cu) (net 28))
 (segment (start 113.03 87.63) (end 115.57 85.09) (width 0.6) (layer B.Cu) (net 28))
 (segment (start 115.57 85.09) (end 120.65 85.09) (width 0.6) (layer B.Cu) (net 28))
 (segment (start 110.470294 85.109706) (end 110.49 85.09) (width 0.6) (layer B.Cu) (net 29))
 (segment (start 106.99121 85.109706) (end 110.470294 85.109706) (width 0.6) (layer B.Cu) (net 29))
 (segment (start 110.49 85.09) (end 113.03 85.09) (width 0.6) (layer B.Cu) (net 29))
 (segment (start 113.03 85.09) (end 115.57 82.55) (width 0.6) (layer B.Cu) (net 29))
 (segment (start 115.57 82.55) (end 120.65 82.55) (width 0.6) (layer B.Cu) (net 29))
 (segment (start 110.470294 82.569706) (end 110.49 82.55) (width 0.6) (layer B.Cu) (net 30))
 (segment (start 106.99121 82.569706) (end 110.470294 82.569706) (width 0.6) (layer B.Cu) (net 30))
 (segment (start 110.49 82.55) (end 113.03 82.55) (width 0.6) (layer B.Cu) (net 30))
 (segment (start 113.03 82.55) (end 115.57 80.01) (width 0.6) (layer B.Cu) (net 30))
 (segment (start 115.57 80.01) (end 120.65 80.01) (width 0.6) (layer B.Cu) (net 30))
 (segment (start 110.470294 80.029706) (end 110.49 80.01) (width 0.6) (layer B.Cu) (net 31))
 (segment (start 106.99121 80.029706) (end 110.470294 80.029706) (width 0.6) (layer B.Cu) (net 31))
 (segment (start 110.49 80.01) (end 113.03 80.01) (width 0.6) (layer B.Cu) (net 31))
 (segment (start 113.03 80.01) (end 115.57 77.47) (width 0.6) (layer B.Cu) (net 31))
 (segment (start 115.57 77.47) (end 120.65 77.47) (width 0.6) (layer B.Cu) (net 31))
 (segment (start 110.470294 77.489706) (end 110.49 77.47) (width 0.6) (layer B.Cu) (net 32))
 (segment (start 106.99121 77.489706) (end 110.470294 77.489706) (width 0.6) (layer B.Cu) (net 32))
 (segment (start 110.49 77.47) (end 113.03 77.47) (width 0.6) (layer B.Cu) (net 32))
 (segment (start 113.03 77.47) (end 115.57 74.93) (width 0.6) (layer B.Cu) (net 32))
 (segment (start 115.57 74.93) (end 120.65 74.93) (width 0.6) (layer B.Cu) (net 32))
 (segment (start 110.470294 74.949706) (end 110.49 74.93) (width 0.6) (layer B.Cu) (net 33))
 (segment (start 106.99121 74.949706) (end 110.470294 74.949706) (width 0.6) (layer B.Cu) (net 33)))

